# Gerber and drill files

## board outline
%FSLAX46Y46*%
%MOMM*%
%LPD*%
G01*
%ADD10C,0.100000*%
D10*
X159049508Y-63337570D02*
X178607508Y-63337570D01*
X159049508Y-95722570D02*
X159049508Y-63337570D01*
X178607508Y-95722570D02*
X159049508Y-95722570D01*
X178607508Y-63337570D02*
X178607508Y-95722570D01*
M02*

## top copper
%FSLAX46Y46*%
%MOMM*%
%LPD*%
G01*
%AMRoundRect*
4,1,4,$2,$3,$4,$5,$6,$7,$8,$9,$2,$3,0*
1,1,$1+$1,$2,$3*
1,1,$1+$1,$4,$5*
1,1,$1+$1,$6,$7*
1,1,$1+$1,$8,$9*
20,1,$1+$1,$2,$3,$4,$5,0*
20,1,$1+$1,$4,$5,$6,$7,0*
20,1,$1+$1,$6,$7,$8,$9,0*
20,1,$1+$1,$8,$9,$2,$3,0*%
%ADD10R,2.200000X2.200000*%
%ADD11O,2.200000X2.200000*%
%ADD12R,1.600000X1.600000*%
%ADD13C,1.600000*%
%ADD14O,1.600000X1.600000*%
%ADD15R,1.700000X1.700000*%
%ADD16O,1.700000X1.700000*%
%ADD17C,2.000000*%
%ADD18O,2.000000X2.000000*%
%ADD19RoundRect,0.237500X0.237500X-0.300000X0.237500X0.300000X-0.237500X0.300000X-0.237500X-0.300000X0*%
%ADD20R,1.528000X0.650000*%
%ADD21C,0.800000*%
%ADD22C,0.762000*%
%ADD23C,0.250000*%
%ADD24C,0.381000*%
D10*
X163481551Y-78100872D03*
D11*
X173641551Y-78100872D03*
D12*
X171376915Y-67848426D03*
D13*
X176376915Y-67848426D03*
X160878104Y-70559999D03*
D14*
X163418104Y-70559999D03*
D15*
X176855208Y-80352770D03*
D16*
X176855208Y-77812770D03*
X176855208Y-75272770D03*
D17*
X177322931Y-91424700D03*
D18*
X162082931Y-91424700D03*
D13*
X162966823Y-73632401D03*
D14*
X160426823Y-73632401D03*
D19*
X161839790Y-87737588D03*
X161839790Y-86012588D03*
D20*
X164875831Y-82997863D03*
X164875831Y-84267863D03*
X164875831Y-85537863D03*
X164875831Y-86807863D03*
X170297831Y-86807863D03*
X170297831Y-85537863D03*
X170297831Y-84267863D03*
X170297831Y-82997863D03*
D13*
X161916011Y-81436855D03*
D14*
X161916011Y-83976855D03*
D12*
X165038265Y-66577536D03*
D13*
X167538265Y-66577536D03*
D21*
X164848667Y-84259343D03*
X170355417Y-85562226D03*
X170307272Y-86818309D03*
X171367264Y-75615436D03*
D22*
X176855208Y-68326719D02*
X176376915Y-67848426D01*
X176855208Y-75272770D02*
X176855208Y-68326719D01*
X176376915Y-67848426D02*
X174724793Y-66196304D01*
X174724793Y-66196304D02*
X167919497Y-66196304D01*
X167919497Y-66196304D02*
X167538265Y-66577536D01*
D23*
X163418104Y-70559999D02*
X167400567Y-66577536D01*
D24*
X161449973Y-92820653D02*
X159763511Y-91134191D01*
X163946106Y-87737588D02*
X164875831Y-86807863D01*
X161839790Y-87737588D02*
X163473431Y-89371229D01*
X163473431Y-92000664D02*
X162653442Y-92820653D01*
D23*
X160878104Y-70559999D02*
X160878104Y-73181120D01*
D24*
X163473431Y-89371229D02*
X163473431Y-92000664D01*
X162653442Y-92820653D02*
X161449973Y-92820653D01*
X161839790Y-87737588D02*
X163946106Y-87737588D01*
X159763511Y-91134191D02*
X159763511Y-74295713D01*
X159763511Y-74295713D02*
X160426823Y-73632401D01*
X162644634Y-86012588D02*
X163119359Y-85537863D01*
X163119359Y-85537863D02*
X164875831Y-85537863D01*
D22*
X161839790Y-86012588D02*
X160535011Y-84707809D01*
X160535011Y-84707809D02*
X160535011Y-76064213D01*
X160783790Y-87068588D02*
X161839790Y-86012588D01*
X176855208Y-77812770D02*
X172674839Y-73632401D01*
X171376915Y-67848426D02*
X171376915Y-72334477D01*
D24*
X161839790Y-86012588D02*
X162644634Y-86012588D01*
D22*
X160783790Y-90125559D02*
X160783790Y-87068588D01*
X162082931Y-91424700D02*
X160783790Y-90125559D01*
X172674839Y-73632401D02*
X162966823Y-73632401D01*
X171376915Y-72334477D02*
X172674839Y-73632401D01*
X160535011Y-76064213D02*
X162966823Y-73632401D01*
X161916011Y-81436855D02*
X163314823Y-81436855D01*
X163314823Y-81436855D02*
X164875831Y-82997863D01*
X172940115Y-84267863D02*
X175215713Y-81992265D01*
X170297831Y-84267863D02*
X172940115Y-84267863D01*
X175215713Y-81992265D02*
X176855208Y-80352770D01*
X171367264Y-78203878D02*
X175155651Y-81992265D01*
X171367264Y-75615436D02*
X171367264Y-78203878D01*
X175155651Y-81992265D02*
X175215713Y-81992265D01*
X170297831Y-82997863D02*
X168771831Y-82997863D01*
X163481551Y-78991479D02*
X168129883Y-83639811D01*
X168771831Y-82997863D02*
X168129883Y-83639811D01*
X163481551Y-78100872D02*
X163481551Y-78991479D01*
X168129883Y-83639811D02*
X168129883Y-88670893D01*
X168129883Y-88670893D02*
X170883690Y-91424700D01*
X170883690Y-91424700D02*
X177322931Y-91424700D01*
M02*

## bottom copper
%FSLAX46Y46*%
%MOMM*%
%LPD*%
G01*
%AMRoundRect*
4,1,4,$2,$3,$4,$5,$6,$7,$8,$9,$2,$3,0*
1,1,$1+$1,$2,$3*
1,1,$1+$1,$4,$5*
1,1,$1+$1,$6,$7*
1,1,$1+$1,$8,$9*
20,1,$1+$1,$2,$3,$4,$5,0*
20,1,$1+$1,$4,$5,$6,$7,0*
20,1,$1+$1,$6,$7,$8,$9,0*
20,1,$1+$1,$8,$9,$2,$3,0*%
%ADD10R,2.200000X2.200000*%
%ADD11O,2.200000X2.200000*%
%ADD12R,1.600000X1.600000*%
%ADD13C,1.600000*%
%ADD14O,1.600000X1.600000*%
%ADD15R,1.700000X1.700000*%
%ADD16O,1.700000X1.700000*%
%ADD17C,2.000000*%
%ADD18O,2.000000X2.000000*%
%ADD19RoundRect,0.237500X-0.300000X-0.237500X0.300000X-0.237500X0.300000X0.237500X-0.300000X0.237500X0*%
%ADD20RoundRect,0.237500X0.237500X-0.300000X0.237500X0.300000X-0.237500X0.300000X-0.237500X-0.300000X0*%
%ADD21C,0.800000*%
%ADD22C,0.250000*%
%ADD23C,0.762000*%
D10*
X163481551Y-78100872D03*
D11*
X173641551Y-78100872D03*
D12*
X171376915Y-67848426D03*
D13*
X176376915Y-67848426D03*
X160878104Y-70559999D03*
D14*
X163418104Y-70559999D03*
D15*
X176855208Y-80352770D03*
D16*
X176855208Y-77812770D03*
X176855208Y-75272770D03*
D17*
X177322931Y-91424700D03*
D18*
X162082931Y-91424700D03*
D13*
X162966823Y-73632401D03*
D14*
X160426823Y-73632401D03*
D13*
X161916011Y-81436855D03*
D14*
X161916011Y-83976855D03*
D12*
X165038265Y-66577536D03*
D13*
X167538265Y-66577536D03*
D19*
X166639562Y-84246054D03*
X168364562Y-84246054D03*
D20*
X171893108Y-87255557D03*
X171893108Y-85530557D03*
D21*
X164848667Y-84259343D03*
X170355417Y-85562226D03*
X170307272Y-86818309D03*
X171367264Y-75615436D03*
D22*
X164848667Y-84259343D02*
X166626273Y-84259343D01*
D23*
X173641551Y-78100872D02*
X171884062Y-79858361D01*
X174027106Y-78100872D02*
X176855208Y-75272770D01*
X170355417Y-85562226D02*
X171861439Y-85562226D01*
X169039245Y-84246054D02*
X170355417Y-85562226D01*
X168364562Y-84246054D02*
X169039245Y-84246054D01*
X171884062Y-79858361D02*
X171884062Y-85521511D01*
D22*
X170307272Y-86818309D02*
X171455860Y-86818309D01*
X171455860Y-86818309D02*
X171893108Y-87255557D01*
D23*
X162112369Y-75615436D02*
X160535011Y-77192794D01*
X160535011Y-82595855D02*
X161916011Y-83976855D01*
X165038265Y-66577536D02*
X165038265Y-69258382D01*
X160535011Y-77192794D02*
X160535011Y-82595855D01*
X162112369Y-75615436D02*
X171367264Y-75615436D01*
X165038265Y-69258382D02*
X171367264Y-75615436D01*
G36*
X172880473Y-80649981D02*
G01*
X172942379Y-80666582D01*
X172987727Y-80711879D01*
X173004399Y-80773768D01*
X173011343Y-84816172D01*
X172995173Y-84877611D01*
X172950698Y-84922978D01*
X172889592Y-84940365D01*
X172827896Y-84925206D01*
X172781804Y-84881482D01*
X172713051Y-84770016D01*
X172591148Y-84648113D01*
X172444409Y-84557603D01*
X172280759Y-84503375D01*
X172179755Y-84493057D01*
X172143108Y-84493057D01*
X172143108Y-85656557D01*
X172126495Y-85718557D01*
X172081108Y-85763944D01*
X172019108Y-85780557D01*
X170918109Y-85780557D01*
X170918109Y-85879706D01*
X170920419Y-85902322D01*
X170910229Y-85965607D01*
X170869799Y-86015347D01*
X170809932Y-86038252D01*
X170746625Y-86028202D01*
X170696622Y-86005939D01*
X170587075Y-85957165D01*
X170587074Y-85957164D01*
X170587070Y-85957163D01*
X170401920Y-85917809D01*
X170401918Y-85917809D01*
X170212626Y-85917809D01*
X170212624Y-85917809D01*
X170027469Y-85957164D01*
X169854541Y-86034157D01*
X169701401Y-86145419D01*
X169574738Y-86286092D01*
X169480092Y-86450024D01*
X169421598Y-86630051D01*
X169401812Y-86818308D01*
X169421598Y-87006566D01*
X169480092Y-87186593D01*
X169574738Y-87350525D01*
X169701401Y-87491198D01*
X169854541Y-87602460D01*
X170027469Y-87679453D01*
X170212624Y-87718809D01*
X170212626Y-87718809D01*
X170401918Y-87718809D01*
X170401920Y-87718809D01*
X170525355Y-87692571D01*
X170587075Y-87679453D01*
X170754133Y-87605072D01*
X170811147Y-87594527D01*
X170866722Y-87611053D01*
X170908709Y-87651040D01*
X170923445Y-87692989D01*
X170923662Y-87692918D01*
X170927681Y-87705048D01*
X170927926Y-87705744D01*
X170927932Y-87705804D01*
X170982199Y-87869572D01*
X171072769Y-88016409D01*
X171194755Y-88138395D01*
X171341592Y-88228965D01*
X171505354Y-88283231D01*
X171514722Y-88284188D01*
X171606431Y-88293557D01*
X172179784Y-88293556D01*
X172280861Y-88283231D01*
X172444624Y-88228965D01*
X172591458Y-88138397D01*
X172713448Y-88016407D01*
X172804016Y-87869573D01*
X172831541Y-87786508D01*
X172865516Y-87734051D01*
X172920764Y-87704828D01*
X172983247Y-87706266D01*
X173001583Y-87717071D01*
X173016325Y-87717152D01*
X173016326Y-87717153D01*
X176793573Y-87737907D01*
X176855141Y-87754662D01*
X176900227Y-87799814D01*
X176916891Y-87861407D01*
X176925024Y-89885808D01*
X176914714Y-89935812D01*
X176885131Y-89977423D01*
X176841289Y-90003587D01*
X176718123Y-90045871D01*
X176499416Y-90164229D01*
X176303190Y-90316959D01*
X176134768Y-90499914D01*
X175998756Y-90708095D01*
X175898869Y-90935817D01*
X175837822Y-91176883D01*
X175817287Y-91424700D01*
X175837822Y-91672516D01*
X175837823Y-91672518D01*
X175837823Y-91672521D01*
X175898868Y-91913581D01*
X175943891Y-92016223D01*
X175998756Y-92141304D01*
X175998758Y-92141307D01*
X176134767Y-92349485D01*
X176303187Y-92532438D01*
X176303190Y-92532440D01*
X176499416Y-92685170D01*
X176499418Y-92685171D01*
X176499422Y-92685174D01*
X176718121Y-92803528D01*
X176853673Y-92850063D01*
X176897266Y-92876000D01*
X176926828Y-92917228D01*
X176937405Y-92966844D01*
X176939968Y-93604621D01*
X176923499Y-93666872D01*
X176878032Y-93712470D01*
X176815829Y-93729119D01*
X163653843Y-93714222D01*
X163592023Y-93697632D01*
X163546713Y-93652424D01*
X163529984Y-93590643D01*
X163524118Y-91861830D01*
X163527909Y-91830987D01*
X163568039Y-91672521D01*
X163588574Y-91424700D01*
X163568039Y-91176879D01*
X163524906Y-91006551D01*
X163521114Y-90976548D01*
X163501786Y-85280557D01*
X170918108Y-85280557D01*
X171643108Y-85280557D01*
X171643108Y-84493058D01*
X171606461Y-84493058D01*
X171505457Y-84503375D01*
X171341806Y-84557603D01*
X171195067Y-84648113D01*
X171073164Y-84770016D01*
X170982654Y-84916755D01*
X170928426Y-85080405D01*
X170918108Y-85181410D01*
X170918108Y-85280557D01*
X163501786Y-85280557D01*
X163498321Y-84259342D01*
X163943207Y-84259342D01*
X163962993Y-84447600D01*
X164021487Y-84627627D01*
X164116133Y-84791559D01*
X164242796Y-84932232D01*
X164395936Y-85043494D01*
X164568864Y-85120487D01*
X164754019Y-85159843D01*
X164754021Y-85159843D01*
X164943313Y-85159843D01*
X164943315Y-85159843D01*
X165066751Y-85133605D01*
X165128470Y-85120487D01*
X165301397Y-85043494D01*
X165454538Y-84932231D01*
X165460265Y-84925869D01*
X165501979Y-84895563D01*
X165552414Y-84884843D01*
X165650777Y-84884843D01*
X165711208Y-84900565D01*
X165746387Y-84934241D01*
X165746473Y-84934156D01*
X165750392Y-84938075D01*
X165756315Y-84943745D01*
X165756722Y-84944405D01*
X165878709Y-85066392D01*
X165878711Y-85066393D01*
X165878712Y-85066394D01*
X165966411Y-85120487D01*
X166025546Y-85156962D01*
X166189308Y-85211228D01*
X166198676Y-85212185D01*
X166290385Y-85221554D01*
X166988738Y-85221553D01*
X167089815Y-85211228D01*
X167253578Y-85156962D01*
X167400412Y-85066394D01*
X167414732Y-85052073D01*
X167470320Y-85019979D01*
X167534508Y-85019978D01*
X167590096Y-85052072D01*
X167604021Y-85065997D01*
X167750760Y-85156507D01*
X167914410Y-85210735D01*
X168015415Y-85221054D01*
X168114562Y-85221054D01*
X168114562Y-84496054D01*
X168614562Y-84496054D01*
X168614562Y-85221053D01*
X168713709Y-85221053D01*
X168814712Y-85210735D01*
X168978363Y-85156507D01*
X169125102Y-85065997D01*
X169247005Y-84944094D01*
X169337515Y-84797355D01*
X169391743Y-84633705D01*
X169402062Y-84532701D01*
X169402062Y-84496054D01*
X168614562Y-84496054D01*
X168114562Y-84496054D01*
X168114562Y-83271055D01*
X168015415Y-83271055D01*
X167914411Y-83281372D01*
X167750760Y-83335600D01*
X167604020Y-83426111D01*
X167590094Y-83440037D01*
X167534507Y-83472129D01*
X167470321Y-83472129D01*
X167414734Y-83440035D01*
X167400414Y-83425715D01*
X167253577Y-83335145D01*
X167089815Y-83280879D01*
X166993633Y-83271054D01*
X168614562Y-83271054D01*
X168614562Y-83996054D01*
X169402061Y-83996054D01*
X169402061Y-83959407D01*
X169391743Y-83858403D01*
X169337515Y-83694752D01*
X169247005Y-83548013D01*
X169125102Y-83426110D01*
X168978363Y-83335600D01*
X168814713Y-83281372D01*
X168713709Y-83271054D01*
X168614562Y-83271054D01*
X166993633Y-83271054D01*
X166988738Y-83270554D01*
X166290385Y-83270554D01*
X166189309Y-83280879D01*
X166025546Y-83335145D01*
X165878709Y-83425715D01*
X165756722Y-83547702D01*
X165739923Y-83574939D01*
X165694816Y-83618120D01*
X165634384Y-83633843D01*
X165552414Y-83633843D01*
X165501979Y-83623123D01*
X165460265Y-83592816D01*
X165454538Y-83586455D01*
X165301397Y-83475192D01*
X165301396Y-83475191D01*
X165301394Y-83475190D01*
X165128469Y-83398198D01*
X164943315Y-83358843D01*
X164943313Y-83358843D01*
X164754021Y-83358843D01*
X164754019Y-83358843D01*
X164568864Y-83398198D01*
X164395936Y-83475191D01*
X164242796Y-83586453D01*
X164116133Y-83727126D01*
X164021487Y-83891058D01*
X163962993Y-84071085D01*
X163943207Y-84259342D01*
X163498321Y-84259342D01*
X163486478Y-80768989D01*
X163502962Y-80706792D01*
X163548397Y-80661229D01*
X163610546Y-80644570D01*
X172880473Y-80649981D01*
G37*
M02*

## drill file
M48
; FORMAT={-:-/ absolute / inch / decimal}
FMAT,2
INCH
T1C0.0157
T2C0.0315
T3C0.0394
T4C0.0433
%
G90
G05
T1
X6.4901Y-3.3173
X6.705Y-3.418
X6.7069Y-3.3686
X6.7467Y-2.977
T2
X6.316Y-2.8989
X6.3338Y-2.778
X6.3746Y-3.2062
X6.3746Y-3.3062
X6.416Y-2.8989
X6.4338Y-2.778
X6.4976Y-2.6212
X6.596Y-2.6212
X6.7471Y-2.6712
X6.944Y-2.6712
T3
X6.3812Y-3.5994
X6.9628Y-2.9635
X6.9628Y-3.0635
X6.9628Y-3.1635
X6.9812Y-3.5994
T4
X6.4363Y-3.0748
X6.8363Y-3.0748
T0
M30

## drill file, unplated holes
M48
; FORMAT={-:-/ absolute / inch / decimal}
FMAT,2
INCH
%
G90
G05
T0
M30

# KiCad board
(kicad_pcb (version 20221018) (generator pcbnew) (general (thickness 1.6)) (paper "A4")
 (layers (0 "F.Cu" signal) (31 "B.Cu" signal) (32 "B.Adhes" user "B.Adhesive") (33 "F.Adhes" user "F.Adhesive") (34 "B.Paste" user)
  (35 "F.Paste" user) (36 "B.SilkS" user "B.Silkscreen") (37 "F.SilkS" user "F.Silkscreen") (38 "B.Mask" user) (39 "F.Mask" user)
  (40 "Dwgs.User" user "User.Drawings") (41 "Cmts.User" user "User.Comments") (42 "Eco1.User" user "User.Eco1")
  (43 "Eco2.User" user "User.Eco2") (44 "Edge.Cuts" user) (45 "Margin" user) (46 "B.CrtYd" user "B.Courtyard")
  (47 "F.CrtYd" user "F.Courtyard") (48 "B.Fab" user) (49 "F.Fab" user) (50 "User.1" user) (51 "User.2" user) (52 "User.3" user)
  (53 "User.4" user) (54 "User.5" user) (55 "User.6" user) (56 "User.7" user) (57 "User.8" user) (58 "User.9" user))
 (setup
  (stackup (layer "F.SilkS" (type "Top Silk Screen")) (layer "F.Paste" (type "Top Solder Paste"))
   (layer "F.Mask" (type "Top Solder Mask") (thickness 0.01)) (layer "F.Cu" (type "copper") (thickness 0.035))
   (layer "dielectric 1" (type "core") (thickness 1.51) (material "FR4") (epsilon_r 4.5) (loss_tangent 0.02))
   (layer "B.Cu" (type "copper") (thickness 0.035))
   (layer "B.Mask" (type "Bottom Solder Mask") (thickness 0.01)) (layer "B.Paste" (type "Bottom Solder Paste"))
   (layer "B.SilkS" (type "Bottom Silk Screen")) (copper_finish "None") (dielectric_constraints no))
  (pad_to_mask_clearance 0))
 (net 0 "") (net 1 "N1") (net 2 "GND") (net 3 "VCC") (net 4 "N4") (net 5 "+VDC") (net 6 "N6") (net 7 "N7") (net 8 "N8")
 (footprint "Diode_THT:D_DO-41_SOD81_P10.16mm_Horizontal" (layer "F.Cu") (at 163.481551 78.100872)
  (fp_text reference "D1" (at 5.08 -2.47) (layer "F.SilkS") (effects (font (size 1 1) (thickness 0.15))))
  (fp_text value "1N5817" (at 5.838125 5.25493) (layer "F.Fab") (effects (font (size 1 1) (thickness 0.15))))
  (pad "1" thru_hole rect (at 0 0) (size 2.2 2.2) (drill 1.1) (layers "*.Cu" "*.Mask") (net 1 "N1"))
  (pad "2" thru_hole oval (at 10.16 0) (size 2.2 2.2) (drill 1.1) (layers "*.Cu" "*.Mask") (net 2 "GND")))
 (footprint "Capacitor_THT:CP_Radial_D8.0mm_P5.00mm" (layer "F.Cu") (at 171.376915 67.848426)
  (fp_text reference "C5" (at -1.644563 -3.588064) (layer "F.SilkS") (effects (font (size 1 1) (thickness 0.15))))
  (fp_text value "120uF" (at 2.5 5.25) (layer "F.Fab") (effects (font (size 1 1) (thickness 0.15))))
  (pad "1" thru_hole rect (at 0 0) (size 1.6 1.6) (drill 0.8) (layers "*.Cu" "*.Mask") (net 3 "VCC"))
  (pad "2" thru_hole circle (at 5 0) (size 1.6 1.6) (drill 0.8) (layers "*.Cu" "*.Mask") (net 2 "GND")))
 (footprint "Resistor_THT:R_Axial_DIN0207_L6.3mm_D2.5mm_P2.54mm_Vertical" (layer "F.Cu") (at 160.878104 70.559999)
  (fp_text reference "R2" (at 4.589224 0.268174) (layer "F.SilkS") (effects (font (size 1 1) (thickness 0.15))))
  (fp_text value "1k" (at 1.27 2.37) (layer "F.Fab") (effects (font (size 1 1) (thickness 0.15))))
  (pad "1" thru_hole circle (at 0 0) (size 1.6 1.6) (drill 0.8) (layers "*.Cu" "*.Mask") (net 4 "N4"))
  (pad "2" thru_hole oval (at 2.54 0) (size 1.6 1.6) (drill 0.8) (layers "*.Cu" "*.Mask") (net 2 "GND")))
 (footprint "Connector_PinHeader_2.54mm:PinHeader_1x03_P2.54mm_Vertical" (layer "F.Cu") (at 176.855208 80.35277 180)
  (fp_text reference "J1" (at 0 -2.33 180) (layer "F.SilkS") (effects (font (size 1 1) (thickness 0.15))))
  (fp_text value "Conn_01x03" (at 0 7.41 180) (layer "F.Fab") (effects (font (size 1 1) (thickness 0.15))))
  (pad "1" thru_hole rect (at 0 0 180) (size 1.7 1.7) (drill 1) (layers "*.Cu" "*.Mask") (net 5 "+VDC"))
  (pad "2" thru_hole oval (at 0 2.54 180) (size 1.7 1.7) (drill 1) (layers "*.Cu" "*.Mask") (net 3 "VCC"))
  (pad "3" thru_hole oval (at 0 5.08 180) (size 1.7 1.7) (drill 1) (layers "*.Cu" "*.Mask") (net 2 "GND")))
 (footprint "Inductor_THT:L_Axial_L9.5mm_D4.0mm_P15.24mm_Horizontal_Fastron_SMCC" (layer "F.Cu") (at 177.322931 91.4247 180)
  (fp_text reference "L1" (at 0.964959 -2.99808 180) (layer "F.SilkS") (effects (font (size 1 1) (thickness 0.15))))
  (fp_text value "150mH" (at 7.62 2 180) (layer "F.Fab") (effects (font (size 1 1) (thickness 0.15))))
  (pad "1" thru_hole circle (at 0 0 180) (size 2 2) (drill 1) (layers "*.Cu" "*.Mask") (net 1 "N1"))
  (pad "2" thru_hole oval (at 15.24 0 180) (size 2 2) (drill 1) (layers "*.Cu" "*.Mask") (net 3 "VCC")))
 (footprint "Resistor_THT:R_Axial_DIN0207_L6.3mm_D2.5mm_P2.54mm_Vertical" (layer "F.Cu") (at 162.966823 73.632401 180)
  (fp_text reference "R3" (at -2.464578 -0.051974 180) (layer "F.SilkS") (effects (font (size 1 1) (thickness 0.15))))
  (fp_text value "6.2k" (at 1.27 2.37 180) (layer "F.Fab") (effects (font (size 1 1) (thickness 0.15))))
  (pad "1" thru_hole circle (at 0 0 180) (size 1.6 1.6) (drill 0.8) (layers "*.Cu" "*.Mask") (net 3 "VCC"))
  (pad "2" thru_hole oval (at 2.54 0 180) (size 1.6 1.6) (drill 0.8) (layers "*.Cu" "*.Mask") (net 4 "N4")))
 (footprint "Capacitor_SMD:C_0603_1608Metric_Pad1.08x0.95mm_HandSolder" (layer "F.Cu") (at 161.83979 86.875088 90)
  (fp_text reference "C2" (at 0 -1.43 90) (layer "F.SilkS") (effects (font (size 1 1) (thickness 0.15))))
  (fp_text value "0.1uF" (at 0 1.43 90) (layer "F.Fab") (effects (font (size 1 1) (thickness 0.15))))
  (pad "1" smd roundrect (at -0.8625 0 90) (size 1.075 0.95) (layers "F.Cu" "F.Paste" "F.Mask") (roundrect_rratio 0.25) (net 4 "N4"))
  (pad "2" smd roundrect (at 0.8625 0 90) (size 1.075 0.95) (layers "F.Cu" "F.Paste" "F.Mask") (roundrect_rratio 0.25) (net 3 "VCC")))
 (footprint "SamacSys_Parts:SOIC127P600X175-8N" (layer "F.Cu") (at 167.586831 84.902863)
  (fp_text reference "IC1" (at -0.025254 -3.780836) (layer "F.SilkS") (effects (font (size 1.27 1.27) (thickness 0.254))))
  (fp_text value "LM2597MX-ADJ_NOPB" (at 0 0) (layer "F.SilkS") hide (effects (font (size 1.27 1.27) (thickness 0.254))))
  (pad "1" smd rect (at -2.711 -1.905 90) (size 0.65 1.528) (layers "F.Cu" "F.Paste" "F.Mask") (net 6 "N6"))
  (pad "2" smd rect (at -2.711 -0.635 90) (size 0.65 1.528) (layers "F.Cu" "F.Paste" "F.Mask") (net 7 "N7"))
  (pad "3" smd rect (at -2.711 0.635 90) (size 0.65 1.528) (layers "F.Cu" "F.Paste" "F.Mask") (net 3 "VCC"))
  (pad "4" smd rect (at -2.711 1.905 90) (size 0.65 1.528) (layers "F.Cu" "F.Paste" "F.Mask") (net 4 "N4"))
  (pad "5" smd rect (at 2.711 1.905 90) (size 0.65 1.528) (layers "F.Cu" "F.Paste" "F.Mask") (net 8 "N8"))
  (pad "6" smd rect (at 2.711 0.635 90) (size 0.65 1.528) (layers "F.Cu" "F.Paste" "F.Mask") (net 2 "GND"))
  (pad "7" smd rect (at 2.711 -0.635 90) (size 0.65 1.528) (layers "F.Cu" "F.Paste" "F.Mask") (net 5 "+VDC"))
  (pad "8" smd rect (at 2.711 -1.905 90) (size 0.65 1.528) (layers "F.Cu" "F.Paste" "F.Mask") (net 1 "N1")))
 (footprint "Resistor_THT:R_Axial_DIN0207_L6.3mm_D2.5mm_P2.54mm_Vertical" (layer "F.Cu") (at 161.916011 81.436855 -90)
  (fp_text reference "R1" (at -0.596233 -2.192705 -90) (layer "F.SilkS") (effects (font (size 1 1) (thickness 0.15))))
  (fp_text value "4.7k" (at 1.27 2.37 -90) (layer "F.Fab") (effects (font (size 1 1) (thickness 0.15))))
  (pad "1" thru_hole circle (at 0 0 270) (size 1.6 1.6) (drill 0.8) (layers "*.Cu" "*.Mask") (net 6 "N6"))
  (pad "2" thru_hole oval (at 2.54 0 270) (size 1.6 1.6) (drill 0.8) (layers "*.Cu" "*.Mask") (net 5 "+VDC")))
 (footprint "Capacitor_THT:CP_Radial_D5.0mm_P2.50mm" (layer "F.Cu") (at 165.038265 66.577536)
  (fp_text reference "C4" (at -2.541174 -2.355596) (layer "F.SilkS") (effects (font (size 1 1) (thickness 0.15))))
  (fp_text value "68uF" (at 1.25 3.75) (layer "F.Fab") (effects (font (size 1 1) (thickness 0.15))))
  (pad "1" thru_hole rect (at 0 0) (size 1.6 1.6) (drill 0.8) (layers "*.Cu" "*.Mask") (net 5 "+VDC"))
  (pad "2" thru_hole circle (at 2.5 0) (size 1.6 1.6) (drill 0.8) (layers "*.Cu" "*.Mask") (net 2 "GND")))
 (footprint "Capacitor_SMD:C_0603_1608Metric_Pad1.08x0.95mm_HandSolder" (layer "B.Cu") (at 167.502062 84.246054)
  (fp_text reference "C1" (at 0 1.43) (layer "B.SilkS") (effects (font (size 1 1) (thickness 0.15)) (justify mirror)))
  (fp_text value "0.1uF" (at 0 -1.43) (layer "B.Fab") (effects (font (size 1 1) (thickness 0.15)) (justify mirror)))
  (pad "1" smd roundrect (at -0.8625 0) (size 1.075 0.95) (layers "B.Cu" "B.Paste" "B.Mask") (roundrect_rratio 0.25) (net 7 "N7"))
  (pad "2" smd roundrect (at 0.8625 0) (size 1.075 0.95) (layers "B.Cu" "B.Paste" "B.Mask") (roundrect_rratio 0.25) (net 2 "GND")))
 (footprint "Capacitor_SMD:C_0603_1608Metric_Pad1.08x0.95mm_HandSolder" (layer "B.Cu") (at 171.893108 86.393057 90)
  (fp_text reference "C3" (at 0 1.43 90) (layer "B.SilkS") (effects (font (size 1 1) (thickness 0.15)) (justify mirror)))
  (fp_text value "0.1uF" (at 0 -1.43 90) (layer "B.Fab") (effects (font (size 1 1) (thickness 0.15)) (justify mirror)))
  (pad "1" smd roundrect (at -0.8625 0 90) (size 1.075 0.95) (layers "B.Cu" "B.Paste" "B.Mask") (roundrect_rratio 0.25) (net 8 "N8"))
  (pad "2" smd roundrect (at 0.8625 0 90) (size 1.075 0.95) (layers "B.Cu" "B.Paste" "B.Mask") (roundrect_rratio 0.25) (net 2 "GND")))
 (gr_line (start 159.049508 63.33757) (end 178.607508 63.33757) (stroke (width 0.1) (type solid)) (layer "Edge.Cuts"))
 (gr_line (start 159.049508 95.72257) (end 159.049508 63.33757) (stroke (width 0.1) (type solid)) (layer "Edge.Cuts"))
 (gr_line (start 178.607508 95.72257) (end 159.049508 95.72257) (stroke (width 0.1) (type default)) (layer "Edge.Cuts"))
 (gr_line (start 178.607508 63.33757) (end 178.607508 95.72257) (stroke (width 0.1) (type default)) (layer "Edge.Cuts"))
 (via (at 164.848667 84.259343) (size 0.8) (drill 0.4) (layers "F.Cu" "B.Cu") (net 7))
 (segment (start 164.848667 84.259343) (end 166.626273 84.259343) (width 0.25) (layer "B.Cu") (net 7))
 (segment (start 176.855208 68.326719) (end 176.376915 67.848426) (width 0.762) (layer "F.Cu") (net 2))
 (segment (start 176.855208 75.27277) (end 176.855208 68.326719) (width 0.762) (layer "F.Cu") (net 2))
 (segment (start 176.376915 67.848426) (end 174.724793 66.196304) (width 0.762) (layer "F.Cu") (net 2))
 (segment (start 174.724793 66.196304) (end 167.919497 66.196304) (width 0.762) (layer "F.Cu") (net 2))
 (segment (start 167.919497 66.196304) (end 167.538265 66.577536) (width 0.762) (layer "F.Cu") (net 2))
 (segment (start 163.418104 70.559999) (end 167.400567 66.577536) (width 0.25) (layer "F.Cu") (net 2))
 (via (at 170.355417 85.562226) (size 0.8) (drill 0.4) (layers "F.Cu" "B.Cu") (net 2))
 (segment (start 173.641551 78.100872) (end 171.884062 79.858361) (width 0.762) (layer "B.Cu") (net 2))
 (segment (start 174.027106 78.100872) (end 176.855208 75.27277) (width 0.762) (layer "B.Cu") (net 2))
 (segment (start 170.355417 85.562226) (end 171.861439 85.562226) (width 0.762) (layer "B.Cu") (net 2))
 (segment (start 169.039245 84.246054) (end 170.355417 85.562226) (width 0.762) (layer "B.Cu") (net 2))
 (segment (start 168.364562 84.246054) (end 169.039245 84.246054) (width 0.762) (layer "B.Cu") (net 2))
 (segment (start 171.884062 79.858361) (end 171.884062 85.521511) (width 0.762) (layer "B.Cu") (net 2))
 (segment (start 161.449973 92.820653) (end 159.763511 91.134191) (width 0.381) (layer "F.Cu") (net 4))
 (segment (start 163.946106 87.737588) (end 164.875831 86.807863) (width 0.381) (layer "F.Cu") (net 4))
 (segment (start 161.83979 87.737588) (end 163.473431 89.371229) (width 0.381) (layer "F.Cu") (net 4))
 (segment (start 163.473431 92.000664) (end 162.653442 92.820653) (width 0.381) (layer "F.Cu") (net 4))
 (segment (start 160.878104 70.559999) (end 160.878104 73.18112) (width 0.25) (layer "F.Cu") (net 4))
 (segment (start 163.473431 89.371229) (end 163.473431 92.000664) (width 0.381) (layer "F.Cu") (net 4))
 (segment (start 162.653442 92.820653) (end 161.449973 92.820653) (width 0.381) (layer "F.Cu") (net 4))
 (segment (start 161.83979 87.737588) (end 163.946106 87.737588) (width 0.381) (layer "F.Cu") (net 4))
 (segment (start 159.763511 91.134191) (end 159.763511 74.295713) (width 0.381) (layer "F.Cu") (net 4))
 (segment (start 159.763511 74.295713) (end 160.426823 73.632401) (width 0.381) (layer "F.Cu") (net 4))
 (segment (start 162.644634 86.012588) (end 163.119359 85.537863) (width 0.381) (layer "F.Cu") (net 3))
 (segment (start 163.119359 85.537863) (end 164.875831 85.537863) (width 0.381) (layer "F.Cu") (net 3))
 (segment (start 161.83979 86.012588) (end 160.535011 84.707809) (width 0.762) (layer "F.Cu") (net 3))
 (segment (start 160.535011 84.707809) (end 160.535011 76.064213) (width 0.762) (layer "F.Cu") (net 3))
 (segment (start 160.78379 87.068588) (end 161.83979 86.012588) (width 0.762) (layer "F.Cu") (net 3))
 (segment (start 176.855208 77.81277) (end 172.674839 73.632401) (width 0.762) (layer "F.Cu") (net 3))
 (segment (start 171.376915 67.848426) (end 171.376915 72.334477) (width 0.762) (layer "F.Cu") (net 3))
 (segment (start 161.83979 86.012588) (end 162.644634 86.012588) (width 0.381) (layer "F.Cu") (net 3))
 (segment (start 160.78379 90.125559) (end 160.78379 87.068588) (width 0.762) (layer "F.Cu") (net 3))
 (segment (start 162.082931 91.4247) (end 160.78379 90.125559) (width 0.762) (layer "F.Cu") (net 3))
 (segment (start 172.674839 73.632401) (end 162.966823 73.632401) (width 0.762) (layer "F.Cu") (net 3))
 (segment (start 171.376915 72.334477) (end 172.674839 73.632401) (width 0.762) (layer "F.Cu") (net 3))
 (segment (start 160.535011 76.064213) (end 162.966823 73.632401) (width 0.762) (layer "F.Cu") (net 3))
 (via (at 170.307272 86.818309) (size 0.8) (drill 0.4) (layers "F.Cu" "B.Cu") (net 8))
 (segment (start 170.307272 86.818309) (end 171.45586 86.818309) (width 0.25) (layer "B.Cu") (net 8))
 (segment (start 171.45586 86.818309) (end 171.893108 87.255557) (width 0.25) (layer "B.Cu") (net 8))
 (segment (start 161.916011 81.436855) (end 163.314823 81.436855) (width 0.762) (layer "F.Cu") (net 6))
 (segment (start 163.314823 81.436855) (end 164.875831 82.997863) (width 0.762) (layer "F.Cu") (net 6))
 (segment (start 172.940115 84.267863) (end 175.215713 81.992265) (width 0.762) (layer "F.Cu") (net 5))
 (segment (start 170.297831 84.267863) (end 172.940115 84.267863) (width 0.762) (layer "F.Cu") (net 5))
 (segment (start 175.215713 81.992265) (end 176.855208 80.35277) (width 0.762) (layer "F.Cu") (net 5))
 (segment (start 171.367264 78.203878) (end 175.155651 81.992265) (width 0.762) (layer "F.Cu") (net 5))
 (segment (start 171.367264 75.615436) (end 171.367264 78.203878) (width 0.762) (layer "F.Cu") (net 5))
 (segment (start 175.155651 81.992265) (end 175.215713 81.992265) (width 0.762) (layer "F.Cu") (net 5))
 (via (at 171.367264 75.615436) (size 0.8) (drill 0.4) (layers "F.Cu" "B.Cu") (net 5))
 (segment (start 162.112369 75.615436) (end 160.535011 77.192794) (width 0.762) (layer "B.Cu") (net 5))
 (segment (start 160.535011 82.595855) (end 161.916011 83.976855) (width 0.762) (layer "B.Cu") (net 5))
 (segment (start 165.038265 66.577536) (end 165.038265 69.258382) (width 0.762) (layer "B.Cu") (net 5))
 (segment (start 160.535011 77.192794) (end 160.535011 82.595855) (width 0.762) (layer "B.Cu") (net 5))
 (segment (start 162.112369 75.615436) (end 171.367264 75.615436) (width 0.762) (layer "B.Cu") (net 5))
 (segment (start 165.038265 69.258382) (end 171.367264 75.615436) (width 0.762) (layer "B.Cu") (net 5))
 (segment (start 170.297831 82.997863) (end 168.771831 82.997863) (width 0.762) (layer "F.Cu") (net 1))
 (segment (start 163.481551 78.991479) (end 168.129883 83.639811) (width 0.762) (layer "F.Cu") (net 1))
 (segment (start 168.771831 82.997863) (end 168.129883 83.639811) (width 0.762) (layer "F.Cu") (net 1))
 (segment (start 163.481551 78.100872) (end 163.481551 78.991479) (width 0.762) (layer "F.Cu") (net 1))
 (segment (start 168.129883 83.639811) (end 168.129883 88.670893) (width 0.762) (layer "F.Cu") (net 1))
 (segment (start 168.129883 88.670893) (end 170.88369 91.4247) (width 0.762) (layer "F.Cu") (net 1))
 (segment (start 170.88369 91.4247) (end 177.322931 91.4247) (width 0.762) (layer "F.Cu") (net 1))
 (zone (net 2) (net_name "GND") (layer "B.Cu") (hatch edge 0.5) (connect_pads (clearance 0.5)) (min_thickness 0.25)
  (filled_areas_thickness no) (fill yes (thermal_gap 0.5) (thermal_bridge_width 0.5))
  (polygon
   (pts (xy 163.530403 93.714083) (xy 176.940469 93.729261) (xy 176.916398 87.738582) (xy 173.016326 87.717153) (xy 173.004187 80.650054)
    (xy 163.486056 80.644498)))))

